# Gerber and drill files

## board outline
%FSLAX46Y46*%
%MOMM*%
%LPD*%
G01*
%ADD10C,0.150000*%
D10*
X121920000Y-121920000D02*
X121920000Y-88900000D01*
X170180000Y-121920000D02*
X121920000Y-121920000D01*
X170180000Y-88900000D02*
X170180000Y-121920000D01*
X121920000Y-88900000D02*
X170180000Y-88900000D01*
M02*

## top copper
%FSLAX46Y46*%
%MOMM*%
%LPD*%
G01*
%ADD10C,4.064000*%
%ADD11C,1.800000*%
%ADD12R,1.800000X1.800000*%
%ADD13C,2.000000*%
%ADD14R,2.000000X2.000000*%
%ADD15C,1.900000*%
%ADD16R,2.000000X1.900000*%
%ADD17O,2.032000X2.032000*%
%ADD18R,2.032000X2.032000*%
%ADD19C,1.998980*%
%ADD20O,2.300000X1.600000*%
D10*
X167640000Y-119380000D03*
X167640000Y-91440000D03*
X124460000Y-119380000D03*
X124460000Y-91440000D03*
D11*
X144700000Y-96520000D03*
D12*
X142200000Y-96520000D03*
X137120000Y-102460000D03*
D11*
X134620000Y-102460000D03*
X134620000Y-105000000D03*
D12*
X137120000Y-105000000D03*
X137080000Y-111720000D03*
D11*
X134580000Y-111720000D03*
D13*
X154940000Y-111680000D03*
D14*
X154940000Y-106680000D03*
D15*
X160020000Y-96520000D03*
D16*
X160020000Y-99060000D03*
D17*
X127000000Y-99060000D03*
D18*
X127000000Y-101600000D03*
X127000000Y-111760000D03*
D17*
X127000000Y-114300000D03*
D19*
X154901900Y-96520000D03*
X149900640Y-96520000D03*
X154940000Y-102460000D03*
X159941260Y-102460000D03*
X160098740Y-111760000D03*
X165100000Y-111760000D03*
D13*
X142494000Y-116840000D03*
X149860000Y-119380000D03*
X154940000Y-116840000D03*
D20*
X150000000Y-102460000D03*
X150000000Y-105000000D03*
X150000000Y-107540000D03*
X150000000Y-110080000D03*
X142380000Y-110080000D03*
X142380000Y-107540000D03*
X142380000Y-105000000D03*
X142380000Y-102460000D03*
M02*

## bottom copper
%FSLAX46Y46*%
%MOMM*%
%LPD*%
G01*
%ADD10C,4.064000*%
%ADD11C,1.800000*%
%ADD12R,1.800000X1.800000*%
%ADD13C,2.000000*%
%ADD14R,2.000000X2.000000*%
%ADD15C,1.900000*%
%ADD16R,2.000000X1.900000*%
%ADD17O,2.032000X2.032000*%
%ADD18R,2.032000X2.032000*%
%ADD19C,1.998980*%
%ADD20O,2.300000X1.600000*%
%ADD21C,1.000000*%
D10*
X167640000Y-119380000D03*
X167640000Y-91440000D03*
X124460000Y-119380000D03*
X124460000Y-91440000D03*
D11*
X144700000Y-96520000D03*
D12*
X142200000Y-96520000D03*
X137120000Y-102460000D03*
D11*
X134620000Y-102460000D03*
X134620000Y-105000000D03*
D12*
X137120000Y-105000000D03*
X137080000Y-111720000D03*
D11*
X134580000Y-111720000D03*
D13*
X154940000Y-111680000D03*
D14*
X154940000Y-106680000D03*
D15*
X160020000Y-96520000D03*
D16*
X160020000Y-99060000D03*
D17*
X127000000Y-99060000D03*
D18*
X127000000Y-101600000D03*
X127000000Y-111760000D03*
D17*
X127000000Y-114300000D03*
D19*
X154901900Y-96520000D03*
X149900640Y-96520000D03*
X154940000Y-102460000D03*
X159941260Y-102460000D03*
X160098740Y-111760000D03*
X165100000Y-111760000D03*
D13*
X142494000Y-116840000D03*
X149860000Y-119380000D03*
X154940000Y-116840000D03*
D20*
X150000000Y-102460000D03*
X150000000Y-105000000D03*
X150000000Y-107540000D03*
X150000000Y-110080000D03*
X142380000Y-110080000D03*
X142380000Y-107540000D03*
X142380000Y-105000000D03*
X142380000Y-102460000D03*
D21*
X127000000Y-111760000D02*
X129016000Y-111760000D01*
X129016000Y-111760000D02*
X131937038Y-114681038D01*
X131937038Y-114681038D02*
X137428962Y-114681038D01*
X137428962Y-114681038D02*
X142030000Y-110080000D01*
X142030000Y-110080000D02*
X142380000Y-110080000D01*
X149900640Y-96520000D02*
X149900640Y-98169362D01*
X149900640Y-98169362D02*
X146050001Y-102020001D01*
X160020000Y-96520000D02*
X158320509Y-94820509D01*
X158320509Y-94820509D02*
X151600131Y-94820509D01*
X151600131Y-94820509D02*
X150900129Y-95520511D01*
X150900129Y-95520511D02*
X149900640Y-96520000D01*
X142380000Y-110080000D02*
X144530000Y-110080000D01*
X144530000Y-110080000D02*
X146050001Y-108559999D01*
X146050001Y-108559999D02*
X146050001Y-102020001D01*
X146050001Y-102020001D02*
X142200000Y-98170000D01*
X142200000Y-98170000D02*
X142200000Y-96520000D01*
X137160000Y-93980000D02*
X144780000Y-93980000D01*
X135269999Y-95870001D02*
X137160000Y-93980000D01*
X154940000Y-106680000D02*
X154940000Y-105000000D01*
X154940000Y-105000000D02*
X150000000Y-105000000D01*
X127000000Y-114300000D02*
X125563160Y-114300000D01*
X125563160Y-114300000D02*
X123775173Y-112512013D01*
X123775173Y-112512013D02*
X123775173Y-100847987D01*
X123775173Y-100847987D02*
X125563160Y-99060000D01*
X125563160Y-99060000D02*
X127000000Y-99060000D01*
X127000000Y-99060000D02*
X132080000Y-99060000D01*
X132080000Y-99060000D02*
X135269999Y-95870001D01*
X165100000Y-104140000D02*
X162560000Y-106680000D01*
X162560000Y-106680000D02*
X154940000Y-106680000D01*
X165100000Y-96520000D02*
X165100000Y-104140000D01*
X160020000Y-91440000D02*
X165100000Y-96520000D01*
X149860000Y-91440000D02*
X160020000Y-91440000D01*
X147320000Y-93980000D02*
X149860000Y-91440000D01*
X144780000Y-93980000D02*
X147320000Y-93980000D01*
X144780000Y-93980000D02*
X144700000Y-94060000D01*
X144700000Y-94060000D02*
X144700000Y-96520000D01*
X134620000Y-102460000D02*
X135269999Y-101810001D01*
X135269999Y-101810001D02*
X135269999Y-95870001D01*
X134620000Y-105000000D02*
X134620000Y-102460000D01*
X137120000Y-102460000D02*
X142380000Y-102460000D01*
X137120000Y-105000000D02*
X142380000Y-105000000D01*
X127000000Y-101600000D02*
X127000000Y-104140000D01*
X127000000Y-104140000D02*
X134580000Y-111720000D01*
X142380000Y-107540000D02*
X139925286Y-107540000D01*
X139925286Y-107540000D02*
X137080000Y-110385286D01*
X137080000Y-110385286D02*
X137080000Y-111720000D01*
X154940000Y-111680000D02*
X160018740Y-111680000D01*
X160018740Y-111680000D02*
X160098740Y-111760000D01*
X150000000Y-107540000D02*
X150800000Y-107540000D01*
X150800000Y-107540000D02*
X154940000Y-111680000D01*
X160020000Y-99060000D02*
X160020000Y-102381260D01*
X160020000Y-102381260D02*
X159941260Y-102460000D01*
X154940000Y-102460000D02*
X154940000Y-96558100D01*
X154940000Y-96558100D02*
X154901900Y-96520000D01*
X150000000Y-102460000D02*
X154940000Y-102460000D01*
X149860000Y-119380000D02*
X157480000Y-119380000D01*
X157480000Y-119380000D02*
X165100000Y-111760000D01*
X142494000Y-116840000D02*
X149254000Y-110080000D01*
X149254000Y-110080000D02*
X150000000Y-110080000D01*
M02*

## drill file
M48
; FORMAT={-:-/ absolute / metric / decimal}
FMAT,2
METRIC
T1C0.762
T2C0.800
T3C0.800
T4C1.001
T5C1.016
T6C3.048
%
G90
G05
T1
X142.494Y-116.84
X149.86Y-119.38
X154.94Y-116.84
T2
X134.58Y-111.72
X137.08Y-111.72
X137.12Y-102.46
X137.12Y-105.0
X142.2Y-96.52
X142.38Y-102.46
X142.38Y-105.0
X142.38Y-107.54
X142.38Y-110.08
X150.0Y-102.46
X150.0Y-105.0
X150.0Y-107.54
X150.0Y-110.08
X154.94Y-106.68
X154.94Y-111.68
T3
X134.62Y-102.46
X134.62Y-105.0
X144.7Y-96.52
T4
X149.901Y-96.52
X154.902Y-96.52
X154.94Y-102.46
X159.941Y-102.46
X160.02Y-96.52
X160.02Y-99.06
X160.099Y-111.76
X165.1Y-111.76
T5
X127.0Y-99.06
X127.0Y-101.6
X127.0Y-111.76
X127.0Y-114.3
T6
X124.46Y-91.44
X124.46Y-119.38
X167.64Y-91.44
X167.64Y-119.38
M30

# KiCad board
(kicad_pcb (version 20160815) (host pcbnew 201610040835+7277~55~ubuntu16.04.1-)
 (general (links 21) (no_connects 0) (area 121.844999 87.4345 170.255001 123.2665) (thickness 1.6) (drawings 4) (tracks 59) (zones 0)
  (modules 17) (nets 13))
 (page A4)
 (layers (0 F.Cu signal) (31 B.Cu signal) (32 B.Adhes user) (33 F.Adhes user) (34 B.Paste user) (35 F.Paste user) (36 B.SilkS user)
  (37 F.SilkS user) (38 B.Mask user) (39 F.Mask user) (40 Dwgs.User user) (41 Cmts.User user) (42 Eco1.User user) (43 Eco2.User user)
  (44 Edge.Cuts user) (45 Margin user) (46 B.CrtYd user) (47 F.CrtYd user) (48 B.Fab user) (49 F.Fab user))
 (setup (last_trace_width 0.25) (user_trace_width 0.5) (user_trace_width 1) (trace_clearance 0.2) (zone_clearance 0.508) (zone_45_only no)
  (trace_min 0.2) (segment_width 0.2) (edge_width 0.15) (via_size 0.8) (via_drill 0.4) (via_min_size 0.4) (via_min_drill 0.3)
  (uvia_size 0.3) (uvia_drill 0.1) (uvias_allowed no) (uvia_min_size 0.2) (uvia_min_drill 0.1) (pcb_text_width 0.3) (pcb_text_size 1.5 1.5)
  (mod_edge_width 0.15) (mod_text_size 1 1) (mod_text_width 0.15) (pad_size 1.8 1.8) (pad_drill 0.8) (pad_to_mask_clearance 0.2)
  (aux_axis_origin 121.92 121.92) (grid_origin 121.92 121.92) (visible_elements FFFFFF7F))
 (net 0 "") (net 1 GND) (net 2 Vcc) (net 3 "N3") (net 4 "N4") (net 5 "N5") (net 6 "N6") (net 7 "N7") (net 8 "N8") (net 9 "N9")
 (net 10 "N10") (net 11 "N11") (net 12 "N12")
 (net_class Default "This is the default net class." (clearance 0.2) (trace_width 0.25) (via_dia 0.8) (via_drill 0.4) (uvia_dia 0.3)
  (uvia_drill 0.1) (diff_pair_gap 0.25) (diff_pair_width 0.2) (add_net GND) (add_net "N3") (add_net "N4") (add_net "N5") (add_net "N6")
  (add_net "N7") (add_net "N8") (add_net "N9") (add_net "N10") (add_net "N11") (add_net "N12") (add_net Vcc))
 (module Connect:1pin (layer F.Cu) (at 167.64 119.38)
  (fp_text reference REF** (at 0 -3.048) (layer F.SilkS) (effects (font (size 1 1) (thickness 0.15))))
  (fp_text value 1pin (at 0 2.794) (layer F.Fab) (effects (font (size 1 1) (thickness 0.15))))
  (pad 1 thru_hole circle (at 0 0) (size 4.064 4.064) (drill 3.048) (layers *.Cu *.Mask F.SilkS)))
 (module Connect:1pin (layer F.Cu) (at 167.64 91.44)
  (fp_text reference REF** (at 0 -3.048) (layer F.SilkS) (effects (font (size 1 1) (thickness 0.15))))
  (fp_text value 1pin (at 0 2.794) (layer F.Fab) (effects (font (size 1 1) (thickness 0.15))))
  (pad 1 thru_hole circle (at 0 0) (size 4.064 4.064) (drill 3.048) (layers *.Cu *.Mask F.SilkS)))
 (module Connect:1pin (layer F.Cu) (at 124.46 119.38)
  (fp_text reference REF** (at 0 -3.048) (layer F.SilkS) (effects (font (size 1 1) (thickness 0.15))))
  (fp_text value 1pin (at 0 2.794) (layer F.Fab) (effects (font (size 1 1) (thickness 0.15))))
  (pad 1 thru_hole circle (at 0 0) (size 4.064 4.064) (drill 3.048) (layers *.Cu *.Mask F.SilkS)))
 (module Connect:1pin (layer F.Cu) (at 124.46 91.44)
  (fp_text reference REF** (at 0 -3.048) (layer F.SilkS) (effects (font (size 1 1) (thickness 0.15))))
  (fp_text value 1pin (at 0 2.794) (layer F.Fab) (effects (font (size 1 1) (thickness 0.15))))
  (pad 1 thru_hole circle (at 0 0) (size 4.064 4.064) (drill 3.048) (layers *.Cu *.Mask F.SilkS)))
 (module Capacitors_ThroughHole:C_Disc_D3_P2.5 (layer F.Cu) (at 142.2 96.52)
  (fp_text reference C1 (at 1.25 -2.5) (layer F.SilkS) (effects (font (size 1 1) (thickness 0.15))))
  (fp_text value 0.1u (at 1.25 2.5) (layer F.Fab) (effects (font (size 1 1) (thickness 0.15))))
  (pad 2 thru_hole circle (at 2.5 0) (size 1.8 1.8) (drill 0.8001) (layers *.Cu *.Mask F.SilkS) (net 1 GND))
  (pad 1 thru_hole rect (at 0 0) (size 1.8 1.8) (drill 0.8) (layers *.Cu *.Mask F.SilkS) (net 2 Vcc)))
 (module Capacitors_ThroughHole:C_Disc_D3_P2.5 (layer F.Cu) (at 137.12 102.46 180)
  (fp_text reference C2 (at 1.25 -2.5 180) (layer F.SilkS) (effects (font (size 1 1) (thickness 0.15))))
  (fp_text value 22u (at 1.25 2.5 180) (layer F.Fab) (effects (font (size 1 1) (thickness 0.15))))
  (pad 1 thru_hole rect (at 0 0 180) (size 1.8 1.8) (drill 0.8) (layers *.Cu *.Mask F.SilkS) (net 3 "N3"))
  (pad 2 thru_hole circle (at 2.5 0 180) (size 1.8 1.8) (drill 0.8001) (layers *.Cu *.Mask F.SilkS) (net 1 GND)))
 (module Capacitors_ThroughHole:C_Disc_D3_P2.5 (layer F.Cu) (at 137.12 105 180)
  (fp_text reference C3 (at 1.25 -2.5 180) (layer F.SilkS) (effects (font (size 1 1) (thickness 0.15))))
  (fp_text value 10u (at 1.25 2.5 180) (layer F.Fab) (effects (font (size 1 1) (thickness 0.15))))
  (pad 2 thru_hole circle (at 2.5 0 180) (size 1.8 1.8) (drill 0.8001) (layers *.Cu *.Mask F.SilkS) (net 1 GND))
  (pad 1 thru_hole rect (at 0 0 180) (size 1.8 1.8) (drill 0.8) (layers *.Cu *.Mask F.SilkS) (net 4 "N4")))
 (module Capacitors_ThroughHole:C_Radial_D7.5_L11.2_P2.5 (layer F.Cu) (at 137.08 111.72 180)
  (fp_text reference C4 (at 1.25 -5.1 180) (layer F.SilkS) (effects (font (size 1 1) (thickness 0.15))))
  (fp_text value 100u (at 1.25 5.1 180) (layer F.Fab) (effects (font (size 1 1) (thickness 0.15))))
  (pad 1 thru_hole rect (at 0 0 180) (size 1.8 1.8) (drill 0.8) (layers *.Cu *.Mask F.SilkS) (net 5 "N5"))
  (pad 2 thru_hole circle (at 2.5 0 180) (size 1.8 1.8) (drill 0.8) (layers *.Cu *.Mask F.SilkS) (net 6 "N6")))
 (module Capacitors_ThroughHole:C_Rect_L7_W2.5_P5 (layer F.Cu) (at 154.94 106.68 270)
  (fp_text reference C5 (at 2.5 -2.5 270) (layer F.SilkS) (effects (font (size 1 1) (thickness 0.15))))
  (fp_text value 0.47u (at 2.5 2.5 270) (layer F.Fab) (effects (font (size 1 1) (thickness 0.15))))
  (pad 2 thru_hole circle (at 5 0 270) (size 2 2) (drill 0.8) (layers *.Cu *.Mask F.SilkS) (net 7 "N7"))
  (pad 1 thru_hole rect (at 0 0 270) (size 2 2) (drill 0.8) (layers *.Cu *.Mask F.SilkS) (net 1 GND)))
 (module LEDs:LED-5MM (layer F.Cu) (at 160.02 99.06 90)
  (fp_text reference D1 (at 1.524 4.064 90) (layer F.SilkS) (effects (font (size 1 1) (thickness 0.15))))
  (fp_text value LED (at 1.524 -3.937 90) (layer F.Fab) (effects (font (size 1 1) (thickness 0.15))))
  (pad 2 thru_hole circle (at 2.54 0 90) (size 1.9 1.9) (drill 1.00076) (layers *.Cu *.Mask F.SilkS) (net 2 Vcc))
  (pad 1 thru_hole rect (at 0 0 180) (size 2 1.9) (drill 1.00076) (layers *.Cu *.Mask F.SilkS) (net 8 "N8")))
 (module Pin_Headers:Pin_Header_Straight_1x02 (layer F.Cu) (at 127 101.6 180)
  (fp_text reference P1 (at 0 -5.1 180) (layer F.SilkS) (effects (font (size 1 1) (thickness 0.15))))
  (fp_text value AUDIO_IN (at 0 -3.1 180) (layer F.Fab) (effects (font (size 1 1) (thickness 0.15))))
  (pad 2 thru_hole oval (at 0 2.54 180) (size 2.032 2.032) (drill 1.016) (layers *.Cu *.Mask F.SilkS) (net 1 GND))
  (pad 1 thru_hole rect (at 0 0 180) (size 2.032 2.032) (drill 1.016) (layers *.Cu *.Mask F.SilkS) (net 6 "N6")))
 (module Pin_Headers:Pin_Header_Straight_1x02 (layer F.Cu) (at 127 111.76)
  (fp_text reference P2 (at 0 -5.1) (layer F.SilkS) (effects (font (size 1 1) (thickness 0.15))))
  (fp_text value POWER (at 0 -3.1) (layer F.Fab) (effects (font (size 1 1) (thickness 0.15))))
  (pad 1 thru_hole rect (at 0 0) (size 2.032 2.032) (drill 1.016) (layers *.Cu *.Mask F.SilkS) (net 2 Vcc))
  (pad 2 thru_hole oval (at 0 2.54) (size 2.032 2.032) (drill 1.016) (layers *.Cu *.Mask F.SilkS) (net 1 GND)))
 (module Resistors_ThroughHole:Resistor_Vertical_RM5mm (layer F.Cu) (at 152.4 96.52)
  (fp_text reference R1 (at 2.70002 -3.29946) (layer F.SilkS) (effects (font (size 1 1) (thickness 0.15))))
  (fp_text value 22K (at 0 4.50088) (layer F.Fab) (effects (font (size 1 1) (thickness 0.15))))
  (pad 2 thru_hole circle (at 2.5019 0) (size 1.99898 1.99898) (drill 1.00076) (layers *.Cu *.SilkS *.Mask) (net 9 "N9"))
  (pad 1 thru_hole circle (at -2.49936 0) (size 1.99898 1.99898) (drill 1.00076) (layers *.Cu *.SilkS *.Mask) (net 2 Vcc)))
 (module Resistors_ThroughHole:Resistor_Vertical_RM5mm (layer F.Cu) (at 157.43936 102.46)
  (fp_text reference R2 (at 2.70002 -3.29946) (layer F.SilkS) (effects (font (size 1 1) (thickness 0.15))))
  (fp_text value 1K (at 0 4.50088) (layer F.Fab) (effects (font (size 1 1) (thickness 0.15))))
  (pad 1 thru_hole circle (at -2.49936 0) (size 1.99898 1.99898) (drill 1.00076) (layers *.Cu *.SilkS *.Mask) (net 9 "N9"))
  (pad 2 thru_hole circle (at 2.5019 0) (size 1.99898 1.99898) (drill 1.00076) (layers *.Cu *.SilkS *.Mask) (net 8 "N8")))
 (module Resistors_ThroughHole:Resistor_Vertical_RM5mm (layer F.Cu) (at 162.60064 111.76 180)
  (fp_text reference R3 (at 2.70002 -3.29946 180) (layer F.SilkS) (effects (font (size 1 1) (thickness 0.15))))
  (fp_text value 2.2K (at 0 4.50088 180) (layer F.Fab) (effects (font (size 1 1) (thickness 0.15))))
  (pad 2 thru_hole circle (at 2.5019 0 180) (size 1.99898 1.99898) (drill 1.00076) (layers *.Cu *.SilkS *.Mask) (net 7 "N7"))
  (pad 1 thru_hole circle (at -2.49936 0 180) (size 1.99898 1.99898) (drill 1.00076) (layers *.Cu *.SilkS *.Mask) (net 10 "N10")))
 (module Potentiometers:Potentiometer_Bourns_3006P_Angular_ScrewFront (layer F.Cu) (at 142.494 116.84 180)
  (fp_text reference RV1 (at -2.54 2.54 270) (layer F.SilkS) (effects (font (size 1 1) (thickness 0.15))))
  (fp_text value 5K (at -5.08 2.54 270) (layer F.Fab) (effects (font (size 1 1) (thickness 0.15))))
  (pad 1 thru_hole circle (at 0 0 180) (size 2 2) (drill 0.762) (layers *.Cu *.Mask F.SilkS) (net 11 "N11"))
  (pad 2 thru_hole circle (at -7.366 -2.54 180) (size 2 2) (drill 0.762) (layers *.Cu *.Mask F.SilkS) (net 10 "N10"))
  (pad 3 thru_hole circle (at -12.446 0 180) (size 2 2) (drill 0.762) (layers *.Cu *.Mask F.SilkS) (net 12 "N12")))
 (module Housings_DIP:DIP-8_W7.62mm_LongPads (layer F.Cu) (at 142.38 102.46)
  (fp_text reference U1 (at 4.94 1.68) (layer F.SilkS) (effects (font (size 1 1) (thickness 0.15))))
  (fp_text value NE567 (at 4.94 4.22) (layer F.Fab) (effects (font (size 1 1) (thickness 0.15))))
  (pad 8 thru_hole oval (at 7.62 0) (size 2.3 1.6) (drill 0.8) (layers *.Cu *.Mask F.SilkS) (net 9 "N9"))
  (pad 7 thru_hole oval (at 7.62 2.54) (size 2.3 1.6) (drill 0.8) (layers *.Cu *.Mask F.SilkS) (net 1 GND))
  (pad 6 thru_hole oval (at 7.62 5.08) (size 2.3 1.6) (drill 0.8) (layers *.Cu *.Mask F.SilkS) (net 7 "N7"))
  (pad 5 thru_hole oval (at 7.62 7.62) (size 2.3 1.6) (drill 0.8) (layers *.Cu *.Mask F.SilkS) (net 11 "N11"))
  (pad 4 thru_hole oval (at 0 7.62) (size 2.3 1.6) (drill 0.8) (layers *.Cu *.Mask F.SilkS) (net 2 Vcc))
  (pad 3 thru_hole oval (at 0 5.08) (size 2.3 1.6) (drill 0.8) (layers *.Cu *.Mask F.SilkS) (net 5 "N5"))
  (pad 2 thru_hole oval (at 0 2.54) (size 2.3 1.6) (drill 0.8) (layers *.Cu *.Mask F.SilkS) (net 4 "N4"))
  (pad 1 thru_hole oval (at 0 0) (size 2.3 1.6) (drill 0.8) (layers *.Cu *.Mask F.SilkS) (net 3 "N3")))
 (gr_line (start 121.92 121.92) (end 121.92 88.9) (layer Edge.Cuts) (width 0.15))
 (gr_line (start 170.18 121.92) (end 121.92 121.92) (layer Edge.Cuts) (width 0.15))
 (gr_line (start 170.18 88.9) (end 170.18 121.92) (layer Edge.Cuts) (width 0.15))
 (gr_line (start 121.92 88.9) (end 170.18 88.9) (layer Edge.Cuts) (width 0.15))
 (segment (start 127 111.76) (end 129.016 111.76) (width 1) (layer B.Cu) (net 2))
 (segment (start 129.016 111.76) (end 131.937038 114.681038) (width 1) (layer B.Cu) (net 2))
 (segment (start 131.937038 114.681038) (end 137.428962 114.681038) (width 1) (layer B.Cu) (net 2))
 (segment (start 137.428962 114.681038) (end 142.03 110.08) (width 1) (layer B.Cu) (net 2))
 (segment (start 142.03 110.08) (end 142.38 110.08) (width 1) (layer B.Cu) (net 2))
 (segment (start 149.90064 96.52) (end 149.90064 98.169362) (width 1) (layer B.Cu) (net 2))
 (segment (start 149.90064 98.169362) (end 146.050001 102.020001) (width 1) (layer B.Cu) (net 2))
 (segment (start 160.02 96.52) (end 158.320509 94.820509) (width 1) (layer B.Cu) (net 2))
 (segment (start 158.320509 94.820509) (end 151.600131 94.820509) (width 1) (layer B.Cu) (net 2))
 (segment (start 151.600131 94.820509) (end 150.900129 95.520511) (width 1) (layer B.Cu) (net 2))
 (segment (start 150.900129 95.520511) (end 149.90064 96.52) (width 1) (layer B.Cu) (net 2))
 (segment (start 142.38 110.08) (end 144.53 110.08) (width 1) (layer B.Cu) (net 2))
 (segment (start 144.53 110.08) (end 146.050001 108.559999) (width 1) (layer B.Cu) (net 2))
 (segment (start 146.050001 108.559999) (end 146.050001 102.020001) (width 1) (layer B.Cu) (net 2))
 (segment (start 146.050001 102.020001) (end 142.2 98.17) (width 1) (layer B.Cu) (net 2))
 (segment (start 142.2 98.17) (end 142.2 96.52) (width 1) (layer B.Cu) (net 2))
 (segment (start 137.16 93.98) (end 144.78 93.98) (width 1) (layer B.Cu) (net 1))
 (segment (start 135.269999 95.870001) (end 137.16 93.98) (width 1) (layer B.Cu) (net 1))
 (segment (start 154.94 106.68) (end 154.94 105) (width 1) (layer B.Cu) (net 1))
 (segment (start 154.94 105) (end 150 105) (width 1) (layer B.Cu) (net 1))
 (segment (start 127 114.3) (end 125.56316 114.3) (width 1) (layer B.Cu) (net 1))
 (segment (start 125.56316 114.3) (end 123.775173 112.512013) (width 1) (layer B.Cu) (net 1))
 (segment (start 123.775173 112.512013) (end 123.775173 100.847987) (width 1) (layer B.Cu) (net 1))
 (segment (start 123.775173 100.847987) (end 125.56316 99.06) (width 1) (layer B.Cu) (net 1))
 (segment (start 125.56316 99.06) (end 127 99.06) (width 1) (layer B.Cu) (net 1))
 (segment (start 127 99.06) (end 132.08 99.06) (width 1) (layer B.Cu) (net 1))
 (segment (start 132.08 99.06) (end 135.269999 95.870001) (width 1) (layer B.Cu) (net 1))
 (segment (start 165.1 104.14) (end 162.56 106.68) (width 1) (layer B.Cu) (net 1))
 (segment (start 162.56 106.68) (end 154.94 106.68) (width 1) (layer B.Cu) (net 1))
 (segment (start 165.1 96.52) (end 165.1 104.14) (width 1) (layer B.Cu) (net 1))
 (segment (start 160.02 91.44) (end 165.1 96.52) (width 1) (layer B.Cu) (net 1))
 (segment (start 149.86 91.44) (end 160.02 91.44) (width 1) (layer B.Cu) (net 1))
 (segment (start 147.32 93.98) (end 149.86 91.44) (width 1) (layer B.Cu) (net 1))
 (segment (start 144.78 93.98) (end 147.32 93.98) (width 1) (layer B.Cu) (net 1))
 (segment (start 144.78 93.98) (end 144.7 94.06) (width 1) (layer B.Cu) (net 1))
 (segment (start 144.7 94.06) (end 144.7 96.52) (width 1) (layer B.Cu) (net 1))
 (segment (start 134.62 102.46) (end 135.269999 101.810001) (width 1) (layer B.Cu) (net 1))
 (segment (start 135.269999 101.810001) (end 135.269999 95.870001) (width 1) (layer B.Cu) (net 1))
 (segment (start 134.62 105) (end 134.62 102.46) (width 1) (layer B.Cu) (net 1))
 (segment (start 137.12 102.46) (end 142.38 102.46) (width 1) (layer B.Cu) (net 3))
 (segment (start 137.12 105) (end 142.38 105) (width 1) (layer B.Cu) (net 4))
 (segment (start 127 101.6) (end 127 104.14) (width 1) (layer B.Cu) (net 6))
 (segment (start 127 104.14) (end 134.58 111.72) (width 1) (layer B.Cu) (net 6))
 (segment (start 142.38 107.54) (end 139.925286 107.54) (width 1) (layer B.Cu) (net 5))
 (segment (start 139.925286 107.54) (end 137.08 110.385286) (width 1) (layer B.Cu) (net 5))
 (segment (start 137.08 110.385286) (end 137.08 111.72) (width 1) (layer B.Cu) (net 5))
 (segment (start 154.94 111.68) (end 160.01874 111.68) (width 1) (layer B.Cu) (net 7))
 (segment (start 160.01874 111.68) (end 160.09874 111.76) (width 1) (layer B.Cu) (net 7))
 (segment (start 150 107.54) (end 150.8 107.54) (width 1) (layer B.Cu) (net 7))
 (segment (start 150.8 107.54) (end 154.94 111.68) (width 1) (layer B.Cu) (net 7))
 (segment (start 160.02 99.06) (end 160.02 102.38126) (width 1) (layer B.Cu) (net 8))
 (segment (start 160.02 102.38126) (end 159.94126 102.46) (width 1) (layer B.Cu) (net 8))
 (segment (start 154.94 102.46) (end 154.94 96.5581) (width 1) (layer B.Cu) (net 9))
 (segment (start 154.94 96.5581) (end 154.9019 96.52) (width 1) (layer B.Cu) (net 9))
 (segment (start 150 102.46) (end 154.94 102.46) (width 1) (layer B.Cu) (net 9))
 (segment (start 149.86 119.38) (end 157.48 119.38) (width 1) (layer B.Cu) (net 10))
 (segment (start 157.48 119.38) (end 165.1 111.76) (width 1) (layer B.Cu) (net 10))
 (segment (start 142.494 116.84) (end 149.254 110.08) (width 1) (layer B.Cu) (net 11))
 (segment (start 149.254 110.08) (end 150 110.08) (width 1) (layer B.Cu) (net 11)))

